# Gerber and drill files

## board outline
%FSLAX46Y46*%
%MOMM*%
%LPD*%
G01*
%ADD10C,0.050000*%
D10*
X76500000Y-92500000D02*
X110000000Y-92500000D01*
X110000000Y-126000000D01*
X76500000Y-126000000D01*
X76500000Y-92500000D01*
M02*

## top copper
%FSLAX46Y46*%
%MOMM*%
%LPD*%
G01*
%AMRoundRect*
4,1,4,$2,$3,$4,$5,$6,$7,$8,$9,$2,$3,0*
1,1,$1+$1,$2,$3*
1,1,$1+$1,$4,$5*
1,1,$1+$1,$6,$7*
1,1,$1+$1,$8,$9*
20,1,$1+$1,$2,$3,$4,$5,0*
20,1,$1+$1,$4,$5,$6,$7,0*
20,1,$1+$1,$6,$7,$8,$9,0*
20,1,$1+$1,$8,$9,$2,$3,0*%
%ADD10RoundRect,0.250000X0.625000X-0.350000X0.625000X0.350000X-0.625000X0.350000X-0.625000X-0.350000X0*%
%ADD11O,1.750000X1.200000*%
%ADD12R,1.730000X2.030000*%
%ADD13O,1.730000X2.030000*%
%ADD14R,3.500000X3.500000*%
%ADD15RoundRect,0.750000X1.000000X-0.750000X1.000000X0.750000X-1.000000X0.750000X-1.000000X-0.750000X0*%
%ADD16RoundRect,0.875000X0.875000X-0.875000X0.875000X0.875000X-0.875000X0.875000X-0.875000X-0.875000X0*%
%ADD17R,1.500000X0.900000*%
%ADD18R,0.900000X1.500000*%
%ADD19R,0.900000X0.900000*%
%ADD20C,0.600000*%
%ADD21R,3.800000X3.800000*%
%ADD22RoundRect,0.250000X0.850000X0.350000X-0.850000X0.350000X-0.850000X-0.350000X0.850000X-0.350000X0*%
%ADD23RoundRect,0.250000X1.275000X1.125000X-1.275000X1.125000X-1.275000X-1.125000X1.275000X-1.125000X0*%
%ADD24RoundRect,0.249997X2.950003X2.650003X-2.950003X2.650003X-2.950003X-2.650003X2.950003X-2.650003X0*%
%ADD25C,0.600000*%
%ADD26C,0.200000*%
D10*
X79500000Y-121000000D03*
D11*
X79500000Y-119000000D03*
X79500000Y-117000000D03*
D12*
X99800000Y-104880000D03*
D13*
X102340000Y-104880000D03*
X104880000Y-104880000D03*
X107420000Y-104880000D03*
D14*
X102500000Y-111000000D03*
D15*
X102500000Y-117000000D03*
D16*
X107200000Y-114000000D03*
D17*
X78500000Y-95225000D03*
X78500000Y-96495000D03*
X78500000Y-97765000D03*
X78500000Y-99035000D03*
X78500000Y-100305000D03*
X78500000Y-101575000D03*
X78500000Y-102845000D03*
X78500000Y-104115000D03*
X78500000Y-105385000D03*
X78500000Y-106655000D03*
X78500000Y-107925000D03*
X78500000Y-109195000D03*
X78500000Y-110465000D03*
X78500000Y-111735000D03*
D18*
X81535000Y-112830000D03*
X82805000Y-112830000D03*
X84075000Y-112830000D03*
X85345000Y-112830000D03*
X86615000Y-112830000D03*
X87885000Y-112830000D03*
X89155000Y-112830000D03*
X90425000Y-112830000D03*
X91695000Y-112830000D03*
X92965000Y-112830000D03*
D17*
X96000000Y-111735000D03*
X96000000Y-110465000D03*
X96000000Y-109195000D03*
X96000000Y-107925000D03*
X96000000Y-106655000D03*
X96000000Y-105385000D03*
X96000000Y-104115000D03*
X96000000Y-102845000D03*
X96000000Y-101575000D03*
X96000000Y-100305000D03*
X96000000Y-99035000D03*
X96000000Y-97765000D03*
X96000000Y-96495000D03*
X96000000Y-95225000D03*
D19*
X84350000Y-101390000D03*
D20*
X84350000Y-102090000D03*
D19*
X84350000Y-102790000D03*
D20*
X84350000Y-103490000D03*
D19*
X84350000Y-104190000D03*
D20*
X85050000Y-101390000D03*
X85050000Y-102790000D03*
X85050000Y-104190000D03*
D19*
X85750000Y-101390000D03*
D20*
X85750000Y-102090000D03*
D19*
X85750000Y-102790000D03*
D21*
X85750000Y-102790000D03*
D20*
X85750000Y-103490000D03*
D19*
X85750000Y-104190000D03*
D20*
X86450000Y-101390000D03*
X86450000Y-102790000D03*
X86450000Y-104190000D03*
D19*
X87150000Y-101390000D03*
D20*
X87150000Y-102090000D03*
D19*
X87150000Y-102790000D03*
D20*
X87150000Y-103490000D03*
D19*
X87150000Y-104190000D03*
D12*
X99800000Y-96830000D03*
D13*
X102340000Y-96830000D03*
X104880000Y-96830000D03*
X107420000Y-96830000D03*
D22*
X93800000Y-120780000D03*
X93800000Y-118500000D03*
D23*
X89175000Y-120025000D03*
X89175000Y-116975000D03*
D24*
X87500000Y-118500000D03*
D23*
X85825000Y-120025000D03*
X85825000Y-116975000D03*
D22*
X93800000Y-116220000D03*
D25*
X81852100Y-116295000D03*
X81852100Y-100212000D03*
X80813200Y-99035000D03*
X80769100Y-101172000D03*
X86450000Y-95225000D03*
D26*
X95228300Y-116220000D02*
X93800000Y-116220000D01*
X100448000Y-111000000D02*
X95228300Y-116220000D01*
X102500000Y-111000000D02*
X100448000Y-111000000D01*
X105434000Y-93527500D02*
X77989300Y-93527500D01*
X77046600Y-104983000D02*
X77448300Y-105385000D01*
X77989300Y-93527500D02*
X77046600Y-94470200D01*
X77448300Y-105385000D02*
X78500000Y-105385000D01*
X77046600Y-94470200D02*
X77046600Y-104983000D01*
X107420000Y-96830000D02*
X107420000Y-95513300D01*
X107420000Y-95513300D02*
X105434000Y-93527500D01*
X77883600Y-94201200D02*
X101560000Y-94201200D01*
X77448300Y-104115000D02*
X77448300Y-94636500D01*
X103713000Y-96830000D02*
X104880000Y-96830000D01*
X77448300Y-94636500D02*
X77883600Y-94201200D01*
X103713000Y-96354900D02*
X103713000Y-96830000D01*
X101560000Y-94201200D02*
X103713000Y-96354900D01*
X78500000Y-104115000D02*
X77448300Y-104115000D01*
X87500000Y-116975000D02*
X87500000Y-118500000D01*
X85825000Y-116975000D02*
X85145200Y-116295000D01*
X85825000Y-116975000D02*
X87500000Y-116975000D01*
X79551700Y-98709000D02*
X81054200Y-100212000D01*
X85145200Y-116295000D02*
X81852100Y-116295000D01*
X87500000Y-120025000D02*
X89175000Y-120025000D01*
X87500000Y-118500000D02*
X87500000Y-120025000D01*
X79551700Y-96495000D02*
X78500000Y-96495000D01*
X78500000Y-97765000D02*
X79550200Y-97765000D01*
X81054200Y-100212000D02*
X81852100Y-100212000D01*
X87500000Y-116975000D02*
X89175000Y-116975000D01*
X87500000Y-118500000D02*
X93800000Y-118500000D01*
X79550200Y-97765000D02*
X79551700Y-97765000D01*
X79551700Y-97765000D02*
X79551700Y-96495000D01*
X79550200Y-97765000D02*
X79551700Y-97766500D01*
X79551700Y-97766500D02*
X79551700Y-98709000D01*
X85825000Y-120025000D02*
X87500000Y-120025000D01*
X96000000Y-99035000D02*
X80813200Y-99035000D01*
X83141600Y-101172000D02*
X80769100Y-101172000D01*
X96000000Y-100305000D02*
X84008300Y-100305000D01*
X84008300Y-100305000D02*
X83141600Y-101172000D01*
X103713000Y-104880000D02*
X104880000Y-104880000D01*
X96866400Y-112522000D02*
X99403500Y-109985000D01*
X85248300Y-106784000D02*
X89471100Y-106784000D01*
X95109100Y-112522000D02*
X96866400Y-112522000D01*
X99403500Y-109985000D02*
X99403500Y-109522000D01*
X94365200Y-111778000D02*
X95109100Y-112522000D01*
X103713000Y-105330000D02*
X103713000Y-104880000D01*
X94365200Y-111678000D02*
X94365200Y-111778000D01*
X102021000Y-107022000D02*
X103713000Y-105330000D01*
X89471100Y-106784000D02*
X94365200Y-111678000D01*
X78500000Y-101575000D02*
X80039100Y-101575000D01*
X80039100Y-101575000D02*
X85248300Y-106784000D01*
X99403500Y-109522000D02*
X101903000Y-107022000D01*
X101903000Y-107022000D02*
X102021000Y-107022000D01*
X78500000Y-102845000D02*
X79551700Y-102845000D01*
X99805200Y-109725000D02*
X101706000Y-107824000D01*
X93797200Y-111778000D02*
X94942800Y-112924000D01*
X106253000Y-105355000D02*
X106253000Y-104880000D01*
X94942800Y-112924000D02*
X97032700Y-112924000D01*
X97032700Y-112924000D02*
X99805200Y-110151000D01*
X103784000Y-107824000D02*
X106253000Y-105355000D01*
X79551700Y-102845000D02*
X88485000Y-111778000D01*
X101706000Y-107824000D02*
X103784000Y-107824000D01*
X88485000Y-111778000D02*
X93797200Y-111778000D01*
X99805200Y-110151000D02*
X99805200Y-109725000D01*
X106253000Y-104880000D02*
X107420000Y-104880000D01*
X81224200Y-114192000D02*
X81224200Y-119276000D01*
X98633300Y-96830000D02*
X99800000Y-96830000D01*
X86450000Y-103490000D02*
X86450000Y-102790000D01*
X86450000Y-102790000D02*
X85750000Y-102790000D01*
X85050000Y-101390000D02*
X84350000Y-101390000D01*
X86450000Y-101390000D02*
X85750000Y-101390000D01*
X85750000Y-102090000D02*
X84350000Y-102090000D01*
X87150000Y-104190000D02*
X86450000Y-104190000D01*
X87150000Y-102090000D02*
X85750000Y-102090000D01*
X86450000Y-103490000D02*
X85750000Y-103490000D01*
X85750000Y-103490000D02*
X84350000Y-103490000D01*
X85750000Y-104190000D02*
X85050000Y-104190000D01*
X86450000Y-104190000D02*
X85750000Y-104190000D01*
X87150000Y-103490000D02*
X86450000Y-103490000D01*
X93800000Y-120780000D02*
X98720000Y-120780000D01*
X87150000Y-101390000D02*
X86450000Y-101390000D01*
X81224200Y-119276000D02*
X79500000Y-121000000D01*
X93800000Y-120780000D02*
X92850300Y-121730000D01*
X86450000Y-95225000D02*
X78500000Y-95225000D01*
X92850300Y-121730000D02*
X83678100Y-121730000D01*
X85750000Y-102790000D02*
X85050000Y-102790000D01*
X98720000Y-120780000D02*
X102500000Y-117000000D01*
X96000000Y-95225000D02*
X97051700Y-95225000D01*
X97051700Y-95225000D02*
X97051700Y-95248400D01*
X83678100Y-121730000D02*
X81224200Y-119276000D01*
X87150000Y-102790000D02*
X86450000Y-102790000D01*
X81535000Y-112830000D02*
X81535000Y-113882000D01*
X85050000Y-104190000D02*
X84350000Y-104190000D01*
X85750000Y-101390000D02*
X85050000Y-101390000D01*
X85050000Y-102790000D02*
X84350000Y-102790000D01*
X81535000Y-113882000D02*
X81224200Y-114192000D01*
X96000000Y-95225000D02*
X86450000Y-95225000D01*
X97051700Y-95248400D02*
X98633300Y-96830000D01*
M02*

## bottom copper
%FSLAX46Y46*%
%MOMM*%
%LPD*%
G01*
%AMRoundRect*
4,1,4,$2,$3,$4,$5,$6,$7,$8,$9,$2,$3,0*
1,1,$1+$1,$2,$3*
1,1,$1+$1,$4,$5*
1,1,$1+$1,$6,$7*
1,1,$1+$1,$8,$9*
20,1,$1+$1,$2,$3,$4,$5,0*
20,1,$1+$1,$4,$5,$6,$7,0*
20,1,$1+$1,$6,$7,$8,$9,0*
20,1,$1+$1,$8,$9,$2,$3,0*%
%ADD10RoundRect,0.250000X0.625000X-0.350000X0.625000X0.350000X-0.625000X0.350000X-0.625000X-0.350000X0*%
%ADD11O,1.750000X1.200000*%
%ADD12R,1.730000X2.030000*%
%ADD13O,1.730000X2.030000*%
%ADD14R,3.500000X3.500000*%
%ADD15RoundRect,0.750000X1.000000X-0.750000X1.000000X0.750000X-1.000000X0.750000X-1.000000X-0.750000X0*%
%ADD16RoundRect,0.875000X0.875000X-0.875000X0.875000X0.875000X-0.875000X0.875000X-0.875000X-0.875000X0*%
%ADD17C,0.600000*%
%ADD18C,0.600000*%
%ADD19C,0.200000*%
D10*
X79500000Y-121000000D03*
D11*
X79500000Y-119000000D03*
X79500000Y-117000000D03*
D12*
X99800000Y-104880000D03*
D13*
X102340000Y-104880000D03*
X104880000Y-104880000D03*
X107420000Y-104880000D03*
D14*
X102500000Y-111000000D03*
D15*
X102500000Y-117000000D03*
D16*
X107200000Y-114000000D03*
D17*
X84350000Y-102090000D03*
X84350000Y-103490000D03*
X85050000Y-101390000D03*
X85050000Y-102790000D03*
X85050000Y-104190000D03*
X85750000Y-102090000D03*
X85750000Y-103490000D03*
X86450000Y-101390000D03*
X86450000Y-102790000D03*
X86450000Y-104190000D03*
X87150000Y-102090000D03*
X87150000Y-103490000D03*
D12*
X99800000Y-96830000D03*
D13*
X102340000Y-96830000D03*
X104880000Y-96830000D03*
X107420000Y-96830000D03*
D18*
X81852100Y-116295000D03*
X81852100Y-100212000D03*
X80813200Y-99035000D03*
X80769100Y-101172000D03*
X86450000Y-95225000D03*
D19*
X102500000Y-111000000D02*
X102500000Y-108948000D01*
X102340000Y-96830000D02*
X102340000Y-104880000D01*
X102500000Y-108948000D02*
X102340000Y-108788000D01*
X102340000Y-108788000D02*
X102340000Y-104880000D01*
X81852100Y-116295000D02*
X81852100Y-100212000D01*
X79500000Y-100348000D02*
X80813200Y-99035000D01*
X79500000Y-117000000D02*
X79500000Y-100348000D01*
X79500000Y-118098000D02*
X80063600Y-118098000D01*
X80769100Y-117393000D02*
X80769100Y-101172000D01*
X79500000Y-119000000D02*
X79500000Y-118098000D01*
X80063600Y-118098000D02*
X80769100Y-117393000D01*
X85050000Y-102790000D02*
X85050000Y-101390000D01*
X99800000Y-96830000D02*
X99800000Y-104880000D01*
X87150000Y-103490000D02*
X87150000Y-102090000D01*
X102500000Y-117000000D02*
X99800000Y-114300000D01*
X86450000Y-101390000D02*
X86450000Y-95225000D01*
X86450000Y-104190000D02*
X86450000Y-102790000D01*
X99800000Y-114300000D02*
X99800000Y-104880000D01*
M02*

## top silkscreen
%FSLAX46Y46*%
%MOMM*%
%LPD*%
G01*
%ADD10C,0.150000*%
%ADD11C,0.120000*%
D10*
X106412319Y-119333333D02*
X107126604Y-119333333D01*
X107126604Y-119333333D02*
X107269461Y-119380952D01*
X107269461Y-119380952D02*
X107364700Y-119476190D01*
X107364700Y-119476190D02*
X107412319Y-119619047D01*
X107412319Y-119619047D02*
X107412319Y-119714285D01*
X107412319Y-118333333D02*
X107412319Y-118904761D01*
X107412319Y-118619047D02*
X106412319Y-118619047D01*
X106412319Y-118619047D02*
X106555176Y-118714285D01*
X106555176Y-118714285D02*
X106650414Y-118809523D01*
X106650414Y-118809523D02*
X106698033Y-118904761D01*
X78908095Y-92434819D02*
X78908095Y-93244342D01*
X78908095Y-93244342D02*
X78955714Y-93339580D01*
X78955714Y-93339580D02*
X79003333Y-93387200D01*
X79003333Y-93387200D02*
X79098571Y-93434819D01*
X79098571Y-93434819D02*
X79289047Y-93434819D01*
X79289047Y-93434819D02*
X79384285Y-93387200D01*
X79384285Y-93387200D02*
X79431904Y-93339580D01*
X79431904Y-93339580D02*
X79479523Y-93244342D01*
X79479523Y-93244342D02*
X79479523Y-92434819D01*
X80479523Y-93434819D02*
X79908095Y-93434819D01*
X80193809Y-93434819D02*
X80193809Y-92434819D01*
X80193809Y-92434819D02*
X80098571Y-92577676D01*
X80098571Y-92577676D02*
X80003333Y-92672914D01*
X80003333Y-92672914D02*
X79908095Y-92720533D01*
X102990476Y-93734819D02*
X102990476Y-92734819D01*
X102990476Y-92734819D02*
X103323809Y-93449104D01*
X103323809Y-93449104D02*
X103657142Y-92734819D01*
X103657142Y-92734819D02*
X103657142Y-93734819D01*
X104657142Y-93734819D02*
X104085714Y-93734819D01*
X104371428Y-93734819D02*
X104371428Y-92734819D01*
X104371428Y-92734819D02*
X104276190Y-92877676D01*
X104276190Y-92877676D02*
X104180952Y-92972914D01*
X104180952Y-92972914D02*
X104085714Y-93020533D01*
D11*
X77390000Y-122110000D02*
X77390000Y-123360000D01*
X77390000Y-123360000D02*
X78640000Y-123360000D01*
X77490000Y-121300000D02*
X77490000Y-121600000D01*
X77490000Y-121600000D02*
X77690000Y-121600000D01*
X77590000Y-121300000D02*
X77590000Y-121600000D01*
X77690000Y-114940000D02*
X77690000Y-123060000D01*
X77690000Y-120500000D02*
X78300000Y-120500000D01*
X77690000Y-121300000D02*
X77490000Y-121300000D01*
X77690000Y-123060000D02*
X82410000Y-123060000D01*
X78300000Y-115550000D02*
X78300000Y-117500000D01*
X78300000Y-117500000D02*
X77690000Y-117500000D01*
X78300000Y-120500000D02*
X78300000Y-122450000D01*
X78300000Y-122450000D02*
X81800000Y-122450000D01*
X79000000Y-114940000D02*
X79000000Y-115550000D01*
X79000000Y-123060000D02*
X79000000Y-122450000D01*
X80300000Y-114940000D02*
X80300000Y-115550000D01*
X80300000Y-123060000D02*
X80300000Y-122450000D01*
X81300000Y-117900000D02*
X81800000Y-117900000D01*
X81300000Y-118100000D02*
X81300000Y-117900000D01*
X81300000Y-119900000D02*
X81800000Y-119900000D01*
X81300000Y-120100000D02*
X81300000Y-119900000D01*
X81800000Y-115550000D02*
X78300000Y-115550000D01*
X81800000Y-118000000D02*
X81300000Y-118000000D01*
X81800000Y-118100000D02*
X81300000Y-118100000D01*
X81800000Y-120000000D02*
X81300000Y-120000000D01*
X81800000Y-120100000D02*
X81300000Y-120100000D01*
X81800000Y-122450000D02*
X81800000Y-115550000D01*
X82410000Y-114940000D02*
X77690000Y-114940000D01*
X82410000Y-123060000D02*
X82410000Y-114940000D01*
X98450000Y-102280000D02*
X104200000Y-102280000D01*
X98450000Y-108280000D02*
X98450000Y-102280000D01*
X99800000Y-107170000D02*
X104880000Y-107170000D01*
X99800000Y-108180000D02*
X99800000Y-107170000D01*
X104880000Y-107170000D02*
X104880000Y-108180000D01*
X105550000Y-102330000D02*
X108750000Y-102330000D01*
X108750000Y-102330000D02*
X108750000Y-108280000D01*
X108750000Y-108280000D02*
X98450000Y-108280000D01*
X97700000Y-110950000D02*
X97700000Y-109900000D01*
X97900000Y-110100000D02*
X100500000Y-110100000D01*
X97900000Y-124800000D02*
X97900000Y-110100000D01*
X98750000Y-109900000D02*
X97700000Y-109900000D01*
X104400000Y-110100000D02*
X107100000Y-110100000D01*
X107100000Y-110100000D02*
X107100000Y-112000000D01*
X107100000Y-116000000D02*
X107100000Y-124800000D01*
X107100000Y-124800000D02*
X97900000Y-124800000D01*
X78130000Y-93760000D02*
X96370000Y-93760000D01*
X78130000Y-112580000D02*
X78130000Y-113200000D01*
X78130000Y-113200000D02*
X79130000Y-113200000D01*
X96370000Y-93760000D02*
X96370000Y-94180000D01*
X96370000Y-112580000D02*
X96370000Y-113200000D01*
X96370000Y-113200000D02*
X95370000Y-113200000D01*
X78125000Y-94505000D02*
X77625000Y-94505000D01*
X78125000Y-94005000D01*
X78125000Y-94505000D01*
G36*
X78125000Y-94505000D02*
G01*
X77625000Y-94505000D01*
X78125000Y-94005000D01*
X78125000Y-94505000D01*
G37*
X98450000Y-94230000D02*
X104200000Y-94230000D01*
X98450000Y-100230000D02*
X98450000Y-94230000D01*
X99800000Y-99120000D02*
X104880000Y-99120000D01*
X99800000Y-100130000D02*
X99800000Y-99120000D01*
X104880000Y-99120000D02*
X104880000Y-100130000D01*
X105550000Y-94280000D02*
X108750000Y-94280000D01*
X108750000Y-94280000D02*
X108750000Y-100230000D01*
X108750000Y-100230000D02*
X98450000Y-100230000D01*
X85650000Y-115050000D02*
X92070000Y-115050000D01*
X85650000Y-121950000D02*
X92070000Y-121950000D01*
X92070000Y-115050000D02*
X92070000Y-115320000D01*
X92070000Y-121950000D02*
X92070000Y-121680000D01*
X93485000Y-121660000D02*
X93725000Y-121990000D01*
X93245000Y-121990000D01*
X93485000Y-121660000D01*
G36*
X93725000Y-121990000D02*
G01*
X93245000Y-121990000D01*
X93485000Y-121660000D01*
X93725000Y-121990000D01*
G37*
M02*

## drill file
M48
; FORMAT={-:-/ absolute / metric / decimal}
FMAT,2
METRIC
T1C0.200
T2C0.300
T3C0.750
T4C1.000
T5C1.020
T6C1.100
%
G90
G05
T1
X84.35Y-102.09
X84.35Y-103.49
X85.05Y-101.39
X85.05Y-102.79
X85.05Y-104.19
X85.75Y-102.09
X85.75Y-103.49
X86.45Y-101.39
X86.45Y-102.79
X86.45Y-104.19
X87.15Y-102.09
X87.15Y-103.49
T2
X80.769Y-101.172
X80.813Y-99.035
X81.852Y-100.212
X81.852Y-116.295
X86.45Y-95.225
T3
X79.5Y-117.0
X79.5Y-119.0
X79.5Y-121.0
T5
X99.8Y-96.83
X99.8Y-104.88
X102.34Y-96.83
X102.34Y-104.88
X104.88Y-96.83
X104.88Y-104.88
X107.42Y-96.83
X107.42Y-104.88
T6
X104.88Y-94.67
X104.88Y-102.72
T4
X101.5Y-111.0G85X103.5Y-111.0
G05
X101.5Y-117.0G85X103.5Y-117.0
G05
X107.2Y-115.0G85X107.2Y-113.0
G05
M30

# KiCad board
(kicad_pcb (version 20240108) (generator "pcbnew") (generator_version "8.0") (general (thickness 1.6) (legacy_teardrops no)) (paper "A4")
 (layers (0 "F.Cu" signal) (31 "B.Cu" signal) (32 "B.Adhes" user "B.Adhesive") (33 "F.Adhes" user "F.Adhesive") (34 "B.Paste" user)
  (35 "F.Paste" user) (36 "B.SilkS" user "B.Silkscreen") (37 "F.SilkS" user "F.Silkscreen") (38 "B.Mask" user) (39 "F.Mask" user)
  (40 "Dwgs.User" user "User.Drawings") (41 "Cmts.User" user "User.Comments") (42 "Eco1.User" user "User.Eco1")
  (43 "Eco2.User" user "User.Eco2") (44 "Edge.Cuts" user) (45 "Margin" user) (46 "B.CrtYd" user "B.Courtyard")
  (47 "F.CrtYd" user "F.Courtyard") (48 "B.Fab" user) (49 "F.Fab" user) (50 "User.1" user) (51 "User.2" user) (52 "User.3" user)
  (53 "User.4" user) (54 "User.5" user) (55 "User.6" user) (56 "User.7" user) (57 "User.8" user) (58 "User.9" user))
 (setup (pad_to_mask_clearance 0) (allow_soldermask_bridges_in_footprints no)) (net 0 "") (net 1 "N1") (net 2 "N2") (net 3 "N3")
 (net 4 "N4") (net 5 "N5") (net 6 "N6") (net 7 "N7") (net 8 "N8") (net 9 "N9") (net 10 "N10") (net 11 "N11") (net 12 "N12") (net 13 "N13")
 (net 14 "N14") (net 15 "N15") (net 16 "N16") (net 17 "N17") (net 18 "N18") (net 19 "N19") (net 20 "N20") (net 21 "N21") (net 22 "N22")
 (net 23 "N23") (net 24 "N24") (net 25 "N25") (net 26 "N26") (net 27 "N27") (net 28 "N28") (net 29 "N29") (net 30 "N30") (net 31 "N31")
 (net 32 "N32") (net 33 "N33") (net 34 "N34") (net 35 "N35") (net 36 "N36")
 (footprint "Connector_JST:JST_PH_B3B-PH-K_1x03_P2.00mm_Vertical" (layer "F.Cu") (at 79.5 121 90)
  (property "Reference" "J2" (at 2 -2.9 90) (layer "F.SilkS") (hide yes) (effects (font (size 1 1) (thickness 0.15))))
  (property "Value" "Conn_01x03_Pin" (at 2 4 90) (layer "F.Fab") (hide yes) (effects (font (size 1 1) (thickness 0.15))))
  (fp_line (start -1.11 -2.11) (end -2.36 -2.11) (stroke (width 0.12) (type solid)) (layer "F.SilkS"))
  (fp_line (start -2.36 -2.11) (end -2.36 -0.86) (stroke (width 0.12) (type solid)) (layer "F.SilkS"))
  (fp_line (start -0.3 -2.01) (end -0.6 -2.01) (stroke (width 0.12) (type solid)) (layer "F.SilkS"))
  (fp_line (start -0.6 -2.01) (end -0.6 -1.81) (stroke (width 0.12) (type solid)) (layer "F.SilkS"))
  (fp_line (start -0.3 -1.91) (end -0.6 -1.91) (stroke (width 0.12) (type solid)) (layer "F.SilkS"))
  (fp_line (start 6.06 -1.81) (end -2.06 -1.81) (stroke (width 0.12) (type solid)) (layer "F.SilkS"))
  (fp_line (start 0.5 -1.81) (end 0.5 -1.2) (stroke (width 0.12) (type solid)) (layer "F.SilkS"))
  (fp_line (start -0.3 -1.81) (end -0.3 -2.01) (stroke (width 0.12) (type solid)) (layer "F.SilkS"))
  (fp_line (start -2.06 -1.81) (end -2.06 2.91) (stroke (width 0.12) (type solid)) (layer "F.SilkS"))
  (fp_line (start 5.45 -1.2) (end 3.5 -1.2) (stroke (width 0.12) (type solid)) (layer "F.SilkS"))
  (fp_line (start 3.5 -1.2) (end 3.5 -1.81) (stroke (width 0.12) (type solid)) (layer "F.SilkS"))
  (fp_line (start 0.5 -1.2) (end -1.45 -1.2) (stroke (width 0.12) (type solid)) (layer "F.SilkS"))
  (fp_line (start -1.45 -1.2) (end -1.45 2.3) (stroke (width 0.12) (type solid)) (layer "F.SilkS"))
  (fp_line (start 6.06 -0.5) (end 5.45 -0.5) (stroke (width 0.12) (type solid)) (layer "F.SilkS"))
  (fp_line (start -2.06 -0.5) (end -1.45 -0.5) (stroke (width 0.12) (type solid)) (layer "F.SilkS"))
  (fp_line (start 6.06 0.8) (end 5.45 0.8) (stroke (width 0.12) (type solid)) (layer "F.SilkS"))
  (fp_line (start -2.06 0.8) (end -1.45 0.8) (stroke (width 0.12) (type solid)) (layer "F.SilkS"))
  (fp_line (start 3.1 1.8) (end 3.1 2.3) (stroke (width 0.12) (type solid)) (layer "F.SilkS"))
  (fp_line (start 2.9 1.8) (end 3.1 1.8) (stroke (width 0.12) (type solid)) (layer "F.SilkS"))
  (fp_line (start 1.1 1.8) (end 1.1 2.3) (stroke (width 0.12) (type solid)) (layer "F.SilkS"))
  (fp_line (start 0.9 1.8) (end 1.1 1.8) (stroke (width 0.12) (type solid)) (layer "F.SilkS"))
  (fp_line (start 5.45 2.3) (end 5.45 -1.2) (stroke (width 0.12) (type solid)) (layer "F.SilkS"))
  (fp_line (start 3 2.3) (end 3 1.8) (stroke (width 0.12) (type solid)) (layer "F.SilkS"))
  (fp_line (start 2.9 2.3) (end 2.9 1.8) (stroke (width 0.12) (type solid)) (layer "F.SilkS"))
  (fp_line (start 1 2.3) (end 1 1.8) (stroke (width 0.12) (type solid)) (layer "F.SilkS"))
  (fp_line (start 0.9 2.3) (end 0.9 1.8) (stroke (width 0.12) (type solid)) (layer "F.SilkS"))
  (fp_line (start -1.45 2.3) (end 5.45 2.3) (stroke (width 0.12) (type solid)) (layer "F.SilkS"))
  (fp_line (start 6.06 2.91) (end 6.06 -1.81) (stroke (width 0.12) (type solid)) (layer "F.SilkS"))
  (fp_line (start -2.06 2.91) (end 6.06 2.91) (stroke (width 0.12) (type solid)) (layer "F.SilkS"))
  (pad "1" thru_hole roundrect (at 0 0 90) (size 1.2 1.75) (drill 0.75) (layers "*.Cu" "*.Mask") (remove_unused_layers no)
   (roundrect_rratio 0.208333) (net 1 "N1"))
  (pad "2" thru_hole oval (at 2 0 90) (size 1.2 1.75) (drill 0.75) (layers "*.Cu" "*.Mask") (remove_unused_layers no) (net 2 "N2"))
  (pad "3" thru_hole oval (at 4 0 90) (size 1.2 1.75) (drill 0.75) (layers "*.Cu" "*.Mask") (remove_unused_layers no) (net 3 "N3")))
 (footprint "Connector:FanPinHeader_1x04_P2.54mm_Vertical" (layer "F.Cu") (at 99.8 104.88)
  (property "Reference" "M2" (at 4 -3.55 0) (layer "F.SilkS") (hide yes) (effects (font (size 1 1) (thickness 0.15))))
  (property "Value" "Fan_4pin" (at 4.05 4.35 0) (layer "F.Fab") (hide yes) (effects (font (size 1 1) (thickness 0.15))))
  (fp_line (start -1.35 -2.6) (end 4.4 -2.6) (stroke (width 0.12) (type solid)) (layer "F.SilkS"))
  (fp_line (start -1.35 3.4) (end -1.35 -2.6) (stroke (width 0.12) (type solid)) (layer "F.SilkS"))
  (fp_line (start 0 2.29) (end 5.08 2.29) (stroke (width 0.12) (type solid)) (layer "F.SilkS"))
  (fp_line (start 0 3.3) (end 0 2.29) (stroke (width 0.12) (type solid)) (layer "F.SilkS"))
  (fp_line (start 5.08 2.29) (end 5.08 3.3) (stroke (width 0.12) (type solid)) (layer "F.SilkS"))
  (fp_line (start 5.75 -2.55) (end 8.95 -2.55) (stroke (width 0.12) (type solid)) (layer "F.SilkS"))
  (fp_line (start 8.95 -2.55) (end 8.95 3.4) (stroke (width 0.12) (type solid)) (layer "F.SilkS"))
  (fp_line (start 8.95 3.4) (end -1.35 3.4) (stroke (width 0.12) (type solid)) (layer "F.SilkS"))
  (pad "" np_thru_hole circle (at 5.08 -2.16 90) (size 1.1 1.1) (drill 1.1) (layers "*.Cu" "*.Mask"))
  (pad "1" thru_hole rect (at 0 0 90) (size 2.03 1.73) (drill 1.02) (layers "*.Cu" "*.Mask") (remove_unused_layers no) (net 1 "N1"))
  (pad "2" thru_hole oval (at 2.54 0 90) (size 2.03 1.73) (drill 1.02) (layers "*.Cu" "*.Mask") (remove_unused_layers no) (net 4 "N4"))
  (pad "3" thru_hole oval (at 5.08 0 90) (size 2.03 1.73) (drill 1.02) (layers "*.Cu" "*.Mask") (remove_unused_layers no) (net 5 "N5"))
  (pad "4" thru_hole oval (at 7.62 0 90) (size 2.03 1.73) (drill 1.02) (layers "*.Cu" "*.Mask") (remove_unused_layers no) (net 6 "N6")))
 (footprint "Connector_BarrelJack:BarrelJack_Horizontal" (layer "F.Cu") (at 102.5 111 90)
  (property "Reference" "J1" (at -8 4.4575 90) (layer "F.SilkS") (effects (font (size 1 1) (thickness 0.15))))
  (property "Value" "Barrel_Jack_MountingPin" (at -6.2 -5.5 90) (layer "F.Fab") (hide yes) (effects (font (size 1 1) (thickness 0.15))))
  (fp_line (start 0.05 -4.8) (end 1.1 -4.8) (stroke (width 0.12) (type solid)) (layer "F.SilkS"))
  (fp_line (start 0.9 -4.6) (end 0.9 -2) (stroke (width 0.12) (type solid)) (layer "F.SilkS"))
  (fp_line (start -13.8 -4.6) (end 0.9 -4.6) (stroke (width 0.12) (type solid)) (layer "F.SilkS"))
  (fp_line (start 1.1 -3.75) (end 1.1 -4.8) (stroke (width 0.12) (type solid)) (layer "F.SilkS"))
  (fp_line (start 0.9 1.9) (end 0.9 4.6) (stroke (width 0.12) (type solid)) (layer "F.SilkS"))
  (fp_line (start 0.9 4.6) (end -1 4.6) (stroke (width 0.12) (type solid)) (layer "F.SilkS"))
  (fp_line (start -5 4.6) (end -13.8 4.6) (stroke (width 0.12) (type solid)) (layer "F.SilkS"))
  (fp_line (start -13.8 4.6) (end -13.8 -4.6) (stroke (width 0.12) (type solid)) (layer "F.SilkS"))
  (pad "1" thru_hole rect (at 0 0 90) (size 3.5 3.5) (drill oval 1 3) (layers "*.Cu" "*.Mask") (remove_unused_layers no) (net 4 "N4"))
  (pad "2" thru_hole roundrect (at -6 0 90) (size 3 3.5) (drill oval 1 3) (layers "*.Cu" "*.Mask") (remove_unused_layers no)
   (roundrect_rratio 0.25) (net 1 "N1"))
  (pad "3" thru_hole roundrect (at -3 4.7 90) (size 3.5 3.5) (drill oval 3 1) (layers "*.Cu" "*.Mask") (remove_unused_layers no)
   (roundrect_rratio 0.25)))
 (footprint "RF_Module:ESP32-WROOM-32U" (layer "F.Cu") (at 87.25 103.48)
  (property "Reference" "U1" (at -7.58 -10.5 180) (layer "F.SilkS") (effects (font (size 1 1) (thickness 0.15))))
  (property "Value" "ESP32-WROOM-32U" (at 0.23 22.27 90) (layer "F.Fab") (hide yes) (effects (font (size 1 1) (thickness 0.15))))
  (fp_line (start -9.12 -9.72) (end 9.12 -9.72) (stroke (width 0.12) (type solid)) (layer "F.SilkS"))
  (fp_line (start -9.12 9.1) (end -9.12 9.72) (stroke (width 0.12) (type solid)) (layer "F.SilkS"))
  (fp_line (start -9.12 9.72) (end -8.12 9.72) (stroke (width 0.12) (type solid)) (layer "F.SilkS"))
  (fp_line (start 9.12 -9.72) (end 9.12 -9.3) (stroke (width 0.12) (type solid)) (layer "F.SilkS"))
  (fp_line (start 9.12 9.1) (end 9.12 9.72) (stroke (width 0.12) (type solid)) (layer "F.SilkS"))
  (fp_line (start 9.12 9.72) (end 8.12 9.72) (stroke (width 0.12) (type solid)) (layer "F.SilkS"))
  (fp_poly
   (pts (xy -9.125 -8.975) (xy -9.625 -8.975) (xy -9.125 -9.475) (xy -9.125 -8.975)) (stroke (width 0.12) (type solid)) (fill solid)
   (layer "F.SilkS"))
  (pad "1" smd rect (at -8.75 -8.255) (size 1.5 0.9) (layers "F.Cu" "F.Paste" "F.Mask") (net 1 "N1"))
  (pad "2" smd rect (at -8.75 -6.985) (size 1.5 0.9) (layers "F.Cu" "F.Paste" "F.Mask") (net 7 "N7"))
  (pad "3" smd rect (at -8.75 -5.715) (size 1.5 0.9) (layers "F.Cu" "F.Paste" "F.Mask") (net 7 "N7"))
  (pad "4" smd rect (at -8.75 -4.445) (size 1.5 0.9) (layers "F.Cu" "F.Paste" "F.Mask") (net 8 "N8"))
  (pad "5" smd rect (at -8.75 -3.175) (size 1.5 0.9) (layers "F.Cu" "F.Paste" "F.Mask") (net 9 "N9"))
  (pad "6" smd rect (at -8.75 -1.905) (size 1.5 0.9) (layers "F.Cu" "F.Paste" "F.Mask") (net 5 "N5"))
  (pad "7" smd rect (at -8.75 -0.635) (size 1.5 0.9) (layers "F.Cu" "F.Paste" "F.Mask") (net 6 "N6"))
  (pad "8" smd rect (at -8.75 0.635) (size 1.5 0.9) (layers "F.Cu" "F.Paste" "F.Mask") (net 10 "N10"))
  (pad "9" smd rect (at -8.75 1.905) (size 1.5 0.9) (layers "F.Cu" "F.Paste" "F.Mask") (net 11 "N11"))
  (pad "10" smd rect (at -8.75 3.175) (size 1.5 0.9) (layers "F.Cu" "F.Paste" "F.Mask") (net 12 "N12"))
  (pad "11" smd rect (at -8.75 4.445) (size 1.5 0.9) (layers "F.Cu" "F.Paste" "F.Mask") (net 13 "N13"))
  (pad "12" smd rect (at -8.75 5.715) (size 1.5 0.9) (layers "F.Cu" "F.Paste" "F.Mask") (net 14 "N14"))
  (pad "13" smd rect (at -8.75 6.985) (size 1.5 0.9) (layers "F.Cu" "F.Paste" "F.Mask") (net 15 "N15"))
  (pad "14" smd rect (at -8.75 8.255) (size 1.5 0.9) (layers "F.Cu" "F.Paste" "F.Mask") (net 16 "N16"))
  (pad "15" smd rect (at -5.715 9.35 90) (size 1.5 0.9) (layers "F.Cu" "F.Paste" "F.Mask") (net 1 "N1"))
  (pad "16" smd rect (at -4.445 9.35 90) (size 1.5 0.9) (layers "F.Cu" "F.Paste" "F.Mask") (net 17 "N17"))
  (pad "17" smd rect (at -3.175 9.35 90) (size 1.5 0.9) (layers "F.Cu" "F.Paste" "F.Mask") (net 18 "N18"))
  (pad "18" smd rect (at -1.905 9.35 90) (size 1.5 0.9) (layers "F.Cu" "F.Paste" "F.Mask") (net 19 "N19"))
  (pad "19" smd rect (at -0.635 9.35 90) (size 1.5 0.9) (layers "F.Cu" "F.Paste" "F.Mask") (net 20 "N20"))
  (pad "20" smd rect (at 0.635 9.35 90) (size 1.5 0.9) (layers "F.Cu" "F.Paste" "F.Mask") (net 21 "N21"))
  (pad "21" smd rect (at 1.905 9.35 90) (size 1.5 0.9) (layers "F.Cu" "F.Paste" "F.Mask") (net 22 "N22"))
  (pad "22" smd rect (at 3.175 9.35 90) (size 1.5 0.9) (layers "F.Cu" "F.Paste" "F.Mask") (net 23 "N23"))
  (pad "23" smd rect (at 4.445 9.35 90) (size 1.5 0.9) (layers "F.Cu" "F.Paste" "F.Mask") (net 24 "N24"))
  (pad "24" smd rect (at 5.715 9.35 90) (size 1.5 0.9) (layers "F.Cu" "F.Paste" "F.Mask") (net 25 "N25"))
  (pad "25" smd rect (at 8.75 8.255) (size 1.5 0.9) (layers "F.Cu" "F.Paste" "F.Mask") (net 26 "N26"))
  (pad "26" smd rect (at 8.75 6.985) (size 1.5 0.9) (layers "F.Cu" "F.Paste" "F.Mask") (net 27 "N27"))
  (pad "27" smd rect (at 8.75 5.715) (size 1.5 0.9) (layers "F.Cu" "F.Paste" "F.Mask") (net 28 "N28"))
  (pad "28" smd rect (at 8.75 4.445) (size 1.5 0.9) (layers "F.Cu" "F.Paste" "F.Mask") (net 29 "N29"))
  (pad "29" smd rect (at 8.75 3.175) (size 1.5 0.9) (layers "F.Cu" "F.Paste" "F.Mask") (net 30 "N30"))
  (pad "30" smd rect (at 8.75 1.905) (size 1.5 0.9) (layers "F.Cu" "F.Paste" "F.Mask") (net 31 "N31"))
  (pad "31" smd rect (at 8.75 0.635) (size 1.5 0.9) (layers "F.Cu" "F.Paste" "F.Mask") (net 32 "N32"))
  (pad "32" smd rect (at 8.75 -0.635) (size 1.5 0.9) (layers "F.Cu" "F.Paste" "F.Mask") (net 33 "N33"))
  (pad "33" smd rect (at 8.75 -1.905) (size 1.5 0.9) (layers "F.Cu" "F.Paste" "F.Mask") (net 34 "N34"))
  (pad "34" smd rect (at 8.75 -3.175) (size 1.5 0.9) (layers "F.Cu" "F.Paste" "F.Mask") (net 2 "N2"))
  (pad "35" smd rect (at 8.75 -4.445) (size 1.5 0.9) (layers "F.Cu" "F.Paste" "F.Mask") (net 3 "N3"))
  (pad "36" smd rect (at 8.75 -5.715) (size 1.5 0.9) (layers "F.Cu" "F.Paste" "F.Mask") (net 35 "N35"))
  (pad "37" smd rect (at 8.75 -6.985) (size 1.5 0.9) (layers "F.Cu" "F.Paste" "F.Mask") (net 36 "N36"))
  (pad "38" smd rect (at 8.75 -8.255) (size 1.5 0.9) (layers "F.Cu" "F.Paste" "F.Mask") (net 1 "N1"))
  (pad "39" smd rect (at -2.9 -2.09) (size 0.9 0.9) (layers "F.Cu" "F.Paste") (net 1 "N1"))
  (pad "39" thru_hole circle (at -2.9 -1.39) (size 0.6 0.6) (drill 0.2) (layers "*.Cu" "F.Mask") (remove_unused_layers no) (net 1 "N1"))
  (pad "39" smd rect (at -2.9 -0.69) (size 0.9 0.9) (layers "F.Cu" "F.Paste") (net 1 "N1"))
  (pad "39" thru_hole circle (at -2.9 0.01) (size 0.6 0.6) (drill 0.2) (layers "*.Cu" "F.Mask") (remove_unused_layers no) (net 1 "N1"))
  (pad "39" smd rect (at -2.9 0.71) (size 0.9 0.9) (layers "F.Cu" "F.Paste") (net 1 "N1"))
  (pad "39" thru_hole circle (at -2.2 -2.09) (size 0.6 0.6) (drill 0.2) (layers "*.Cu" "F.Mask") (remove_unused_layers no) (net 1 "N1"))
  (pad "39" thru_hole circle (at -2.2 -0.69) (size 0.6 0.6) (drill 0.2) (layers "*.Cu" "F.Mask") (remove_unused_layers no) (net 1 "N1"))
  (pad "39" thru_hole circle (at -2.2 0.71) (size 0.6 0.6) (drill 0.2) (layers "*.Cu" "F.Mask") (remove_unused_layers no) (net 1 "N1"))
  (pad "39" smd rect (at -1.5 -2.09) (size 0.9 0.9) (layers "F.Cu" "F.Paste") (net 1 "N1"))
  (pad "39" thru_hole circle (at -1.5 -1.39) (size 0.6 0.6) (drill 0.2) (layers "*.Cu" "F.Mask") (remove_unused_layers no) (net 1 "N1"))
  (pad "39" smd rect (at -1.5 -0.69) (size 0.9 0.9) (layers "F.Cu" "F.Paste") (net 1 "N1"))
  (pad "39" smd rect (at -1.5 -0.69) (size 3.8 3.8) (layers "F.Cu" "F.Mask") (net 1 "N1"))
  (pad "39" thru_hole circle (at -1.5 0.01) (size 0.6 0.6) (drill 0.2) (layers "*.Cu" "F.Mask") (remove_unused_layers no) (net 1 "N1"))
  (pad "39" smd rect (at -1.5 0.71) (size 0.9 0.9) (layers "F.Cu" "F.Paste") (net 1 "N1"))
  (pad "39" thru_hole circle (at -0.8 -2.09) (size 0.6 0.6) (drill 0.2) (layers "*.Cu" "F.Mask") (remove_unused_layers no) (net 1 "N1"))
  (pad "39" thru_hole circle (at -0.8 -0.69) (size 0.6 0.6) (drill 0.2) (layers "*.Cu" "F.Mask") (remove_unused_layers no) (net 1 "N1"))
  (pad "39" thru_hole circle (at -0.8 0.71) (size 0.6 0.6) (drill 0.2) (layers "*.Cu" "F.Mask") (remove_unused_layers no) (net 1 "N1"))
  (pad "39" smd rect (at -0.1 -2.09) (size 0.9 0.9) (layers "F.Cu" "F.Paste") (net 1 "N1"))
  (pad "39" thru_hole circle (at -0.1 -1.39) (size 0.6 0.6) (drill 0.2) (layers "*.Cu" "F.Mask") (remove_unused_layers no) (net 1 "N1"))
  (pad "39" smd rect (at -0.1 -0.69) (size 0.9 0.9) (layers "F.Cu" "F.Paste") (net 1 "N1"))
  (pad "39" thru_hole circle (at -0.1 0.01) (size 0.6 0.6) (drill 0.2) (layers "*.Cu" "F.Mask") (remove_unused_layers no) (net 1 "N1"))
  (pad "39" smd rect (at -0.1 0.71) (size 0.9 0.9) (layers "F.Cu" "F.Paste") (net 1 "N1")))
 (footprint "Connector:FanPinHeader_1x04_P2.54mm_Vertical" (layer "F.Cu") (at 99.8 96.83)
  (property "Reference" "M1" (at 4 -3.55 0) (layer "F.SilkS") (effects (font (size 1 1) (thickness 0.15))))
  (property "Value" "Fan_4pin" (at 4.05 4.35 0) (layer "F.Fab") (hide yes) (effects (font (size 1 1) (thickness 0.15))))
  (fp_line (start -1.35 -2.6) (end 4.4 -2.6) (stroke (width 0.12) (type solid)) (layer "F.SilkS"))
  (fp_line (start -1.35 3.4) (end -1.35 -2.6) (stroke (width 0.12) (type solid)) (layer "F.SilkS"))
  (fp_line (start 0 2.29) (end 5.08 2.29) (stroke (width 0.12) (type solid)) (layer "F.SilkS"))
  (fp_line (start 0 3.3) (end 0 2.29) (stroke (width 0.12) (type solid)) (layer "F.SilkS"))
  (fp_line (start 5.08 2.29) (end 5.08 3.3) (stroke (width 0.12) (type solid)) (layer "F.SilkS"))
  (fp_line (start 5.75 -2.55) (end 8.95 -2.55) (stroke (width 0.12) (type solid)) (layer "F.SilkS"))
  (fp_line (start 8.95 -2.55) (end 8.95 3.4) (stroke (width 0.12) (type solid)) (layer "F.SilkS"))
  (fp_line (start 8.95 3.4) (end -1.35 3.4) (stroke (width 0.12) (type solid)) (layer "F.SilkS"))
  (pad "" np_thru_hole circle (at 5.08 -2.16 90) (size 1.1 1.1) (drill 1.1) (layers "*.Cu" "*.Mask"))
  (pad "1" thru_hole rect (at 0 0 90) (size 2.03 1.73) (drill 1.02) (layers "*.Cu" "*.Mask") (remove_unused_layers no) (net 1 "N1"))
  (pad "2" thru_hole oval (at 2.54 0 90) (size 2.03 1.73) (drill 1.02) (layers "*.Cu" "*.Mask") (remove_unused_layers no) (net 4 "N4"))
  (pad "3" thru_hole oval (at 5.08 0 90) (size 2.03 1.73) (drill 1.02) (layers "*.Cu" "*.Mask") (remove_unused_layers no) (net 10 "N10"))
  (pad "4" thru_hole oval (at 7.62 0 90) (size 2.03 1.73) (drill 1.02) (layers "*.Cu" "*.Mask") (remove_unused_layers no) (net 11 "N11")))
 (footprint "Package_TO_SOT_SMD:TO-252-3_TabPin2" (layer "F.Cu") (at 88.76 118.5 180)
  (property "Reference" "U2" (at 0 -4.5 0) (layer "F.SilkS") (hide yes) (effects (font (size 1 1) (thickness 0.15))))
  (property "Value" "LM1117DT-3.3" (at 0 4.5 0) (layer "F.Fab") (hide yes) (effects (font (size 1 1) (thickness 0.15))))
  (fp_line (start 3.11 3.45) (end -3.31 3.45) (stroke (width 0.12) (type solid)) (layer "F.SilkS"))
  (fp_line (start 3.11 -3.45) (end -3.31 -3.45) (stroke (width 0.12) (type solid)) (layer "F.SilkS"))
  (fp_line (start -3.31 3.45) (end -3.31 3.18) (stroke (width 0.12) (type solid)) (layer "F.SilkS"))
  (fp_line (start -3.31 -3.45) (end -3.31 -3.18) (stroke (width 0.12) (type solid)) (layer "F.SilkS"))
  (fp_poly
   (pts (xy -4.725 -3.16) (xy -4.965 -3.49) (xy -4.485 -3.49) (xy -4.725 -3.16)) (stroke (width 0.12) (type solid)) (fill solid)
   (layer "F.SilkS"))
  (pad "1" smd roundrect (at -5.04 -2.28 180) (size 2.2 1.2) (layers "F.Cu" "F.Paste" "F.Mask") (roundrect_rratio 0.208333) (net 1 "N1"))
  (pad "2" smd roundrect (at -5.04 0 180) (size 2.2 1.2) (layers "F.Cu" "F.Paste" "F.Mask") (roundrect_rratio 0.208333) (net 7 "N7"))
  (pad "2" smd roundrect (at -0.415 -1.525 180) (size 3.05 2.75) (layers "F.Cu" "F.Paste") (roundrect_rratio 0.090909) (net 7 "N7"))
  (pad "2" smd roundrect (at -0.415 1.525 180) (size 3.05 2.75) (layers "F.Cu" "F.Paste") (roundrect_rratio 0.090909) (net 7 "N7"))
  (pad "2" smd roundrect (at 1.26 0 180) (size 6.4 5.8) (layers "F.Cu" "F.Mask") (roundrect_rratio 0.043103) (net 7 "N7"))
  (pad "2" smd roundrect (at 2.935 -1.525 180) (size 3.05 2.75) (layers "F.Cu" "F.Paste") (roundrect_rratio 0.090909) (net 7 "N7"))
  (pad "2" smd roundrect (at 2.935 1.525 180) (size 3.05 2.75) (layers "F.Cu" "F.Paste") (roundrect_rratio 0.090909) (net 7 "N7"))
  (pad "3" smd roundrect (at -5.04 2.28 180) (size 2.2 1.2) (layers "F.Cu" "F.Paste" "F.Mask") (roundrect_rratio 0.208333) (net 4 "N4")))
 (gr_rect (start 76.5 92.5) (end 110 126) (stroke (width 0.05) (type default)) (fill none) (layer "Edge.Cuts"))
 (segment (start 95.2283 116.22) (end 93.8 116.22) (width 0.2) (layer "F.Cu") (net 4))
 (segment (start 100.448 111) (end 95.2283 116.22) (width 0.2) (layer "F.Cu") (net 4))
 (segment (start 102.5 111) (end 100.448 111) (width 0.2) (layer "F.Cu") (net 4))
 (segment (start 102.5 111) (end 102.5 108.948) (width 0.2) (layer "B.Cu") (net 4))
 (segment (start 102.34 96.83) (end 102.34 104.88) (width 0.2) (layer "B.Cu") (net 4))
 (segment (start 102.5 108.948) (end 102.34 108.788) (width 0.2) (layer "B.Cu") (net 4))
 (segment (start 102.34 108.788) (end 102.34 104.88) (width 0.2) (layer "B.Cu") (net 4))
 (segment (start 105.434 93.5275) (end 77.9893 93.5275) (width 0.2) (layer "F.Cu") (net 11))
 (segment (start 77.0466 104.983) (end 77.4483 105.385) (width 0.2) (layer "F.Cu") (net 11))
 (segment (start 77.9893 93.5275) (end 77.0466 94.4702) (width 0.2) (layer "F.Cu") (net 11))
 (segment (start 77.4483 105.385) (end 78.5 105.385) (width 0.2) (layer "F.Cu") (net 11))
 (segment (start 77.0466 94.4702) (end 77.0466 104.983) (width 0.2) (layer "F.Cu") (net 11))
 (segment (start 107.42 96.83) (end 107.42 95.5133) (width 0.2) (layer "F.Cu") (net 11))
 (segment (start 107.42 95.5133) (end 105.434 93.5275) (width 0.2) (layer "F.Cu") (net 11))
 (segment (start 77.8836 94.2012) (end 101.56 94.2012) (width 0.2) (layer "F.Cu") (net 10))
 (segment (start 77.4483 104.115) (end 77.4483 94.6365) (width 0.2) (layer "F.Cu") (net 10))
 (segment (start 103.713 96.83) (end 104.88 96.83) (width 0.2) (layer "F.Cu") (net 10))
 (segment (start 77.4483 94.6365) (end 77.8836 94.2012) (width 0.2) (layer "F.Cu") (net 10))
 (segment (start 103.713 96.3549) (end 103.713 96.83) (width 0.2) (layer "F.Cu") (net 10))
 (segment (start 101.56 94.2012) (end 103.713 96.3549) (width 0.2) (layer "F.Cu") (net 10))
 (segment (start 78.5 104.115) (end 77.4483 104.115) (width 0.2) (layer "F.Cu") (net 10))
 (segment (start 87.5 116.975) (end 87.5 118.5) (width 0.2) (layer "F.Cu") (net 7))
 (segment (start 85.825 116.975) (end 85.1452 116.295) (width 0.2) (layer "F.Cu") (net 7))
 (segment (start 85.825 116.975) (end 87.5 116.975) (width 0.2) (layer "F.Cu") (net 7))
 (segment (start 79.5517 98.709) (end 81.0542 100.212) (width 0.2) (layer "F.Cu") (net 7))
 (segment (start 85.1452 116.295) (end 81.8521 116.295) (width 0.2) (layer "F.Cu") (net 7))
 (segment (start 87.5 120.025) (end 89.175 120.025) (width 0.2) (layer "F.Cu") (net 7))
 (segment (start 87.5 118.5) (end 87.5 120.025) (width 0.2) (layer "F.Cu") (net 7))
 (segment (start 79.5517 96.495) (end 78.5 96.495) (width 0.2) (layer "F.Cu") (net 7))
 (segment (start 78.5 97.765) (end 79.5502 97.765) (width 0.2) (layer "F.Cu") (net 7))
 (segment (start 81.0542 100.212) (end 81.8521 100.212) (width 0.2) (layer "F.Cu") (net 7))
 (segment (start 87.5 116.975) (end 89.175 116.975) (width 0.2) (layer "F.Cu") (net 7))
 (segment (start 87.5 118.5) (end 93.8 118.5) (width 0.2) (layer "F.Cu") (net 7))
 (segment (start 79.5502 97.765) (end 79.5517 97.765) (width 0.2) (layer "F.Cu") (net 7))
 (segment (start 79.5517 97.765) (end 79.5517 96.495) (width 0.2) (layer "F.Cu") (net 7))
 (segment (start 79.5502 97.765) (end 79.5517 97.7665) (width 0.2) (layer "F.Cu") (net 7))
 (segment (start 79.5517 97.7665) (end 79.5517 98.709) (width 0.2) (layer "F.Cu") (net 7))
 (segment (start 85.825 120.025) (end 87.5 120.025) (width 0.2) (layer "F.Cu") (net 7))
 (via (at 81.8521 116.295) (size 0.6) (drill 0.3) (layers "F.Cu" "B.Cu") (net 7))
 (via (at 81.8521 100.212) (size 0.6) (drill 0.3) (layers "F.Cu" "B.Cu") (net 7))
 (segment (start 81.8521 116.295) (end 81.8521 100.212) (width 0.2) (layer "B.Cu") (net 7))
 (segment (start 96 99.035) (end 80.8132 99.035) (width 0.2) (layer "F.Cu") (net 3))
 (via (at 80.8132 99.035) (size 0.6) (drill 0.3) (layers "F.Cu" "B.Cu") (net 3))
 (segment (start 79.5 100.348) (end 80.8132 99.035) (width 0.2) (layer "B.Cu") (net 3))
 (segment (start 79.5 117) (end 79.5 100.348) (width 0.2) (layer "B.Cu") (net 3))
 (segment (start 83.1416 101.172) (end 80.7691 101.172) (width 0.2) (layer "F.Cu") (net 2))
 (segment (start 96 100.305) (end 84.0083 100.305) (width 0.2) (layer "F.Cu") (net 2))
 (segment (start 84.0083 100.305) (end 83.1416 101.172) (width 0.2) (layer "F.Cu") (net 2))
 (via (at 80.7691 101.172) (size 0.6) (drill 0.3) (layers "F.Cu" "B.Cu") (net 2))
 (segment (start 79.5 118.098) (end 80.0636 118.098) (width 0.2) (layer "B.Cu") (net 2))
 (segment (start 80.7691 117.393) (end 80.7691 101.172) (width 0.2) (layer "B.Cu") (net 2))
 (segment (start 79.5 119) (end 79.5 118.098) (width 0.2) (layer "B.Cu") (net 2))
 (segment (start 80.0636 118.098) (end 80.7691 117.393) (width 0.2) (layer "B.Cu") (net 2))
 (segment (start 103.713 104.88) (end 104.88 104.88) (width 0.2) (layer "F.Cu") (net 5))
 (segment (start 96.8664 112.522) (end 99.4035 109.985) (width 0.2) (layer "F.Cu") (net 5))
 (segment (start 85.2483 106.784) (end 89.4711 106.784) (width 0.2) (layer "F.Cu") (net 5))
 (segment (start 95.1091 112.522) (end 96.8664 112.522) (width 0.2) (layer "F.Cu") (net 5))
 (segment (start 99.4035 109.985) (end 99.4035 109.522) (width 0.2) (layer "F.Cu") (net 5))
 (segment (start 94.3652 111.778) (end 95.1091 112.522) (width 0.2) (layer "F.Cu") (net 5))
 (segment (start 103.713 105.33) (end 103.713 104.88) (width 0.2) (layer "F.Cu") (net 5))
 (segment (start 94.3652 111.678) (end 94.3652 111.778) (width 0.2) (layer "F.Cu") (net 5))
 (segment (start 102.021 107.022) (end 103.713 105.33) (width 0.2) (layer "F.Cu") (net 5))
 (segment (start 89.4711 106.784) (end 94.3652 111.678) (width 0.2) (layer "F.Cu") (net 5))
 (segment (start 78.5 101.575) (end 80.0391 101.575) (width 0.2) (layer "F.Cu") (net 5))
 (segment (start 80.0391 101.575) (end 85.2483 106.784) (width 0.2) (layer "F.Cu") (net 5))
 (segment (start 99.4035 109.522) (end 101.903 107.022) (width 0.2) (layer "F.Cu") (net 5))
 (segment (start 101.903 107.022) (end 102.021 107.022) (width 0.2) (layer "F.Cu") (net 5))
 (segment (start 78.5 102.845) (end 79.5517 102.845) (width 0.2) (layer "F.Cu") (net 6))
 (segment (start 99.8052 109.725) (end 101.706 107.824) (width 0.2) (layer "F.Cu") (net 6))
 (segment (start 93.7972 111.778) (end 94.9428 112.924) (width 0.2) (layer "F.Cu") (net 6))
 (segment (start 106.253 105.355) (end 106.253 104.88) (width 0.2) (layer "F.Cu") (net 6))
 (segment (start 94.9428 112.924) (end 97.0327 112.924) (width 0.2) (layer "F.Cu") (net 6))
 (segment (start 97.0327 112.924) (end 99.8052 110.151) (width 0.2) (layer "F.Cu") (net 6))
 (segment (start 103.784 107.824) (end 106.253 105.355) (width 0.2) (layer "F.Cu") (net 6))
 (segment (start 79.5517 102.845) (end 88.485 111.778) (width 0.2) (layer "F.Cu") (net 6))
 (segment (start 101.706 107.824) (end 103.784 107.824) (width 0.2) (layer "F.Cu") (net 6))
 (segment (start 88.485 111.778) (end 93.7972 111.778) (width 0.2) (layer "F.Cu") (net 6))
 (segment (start 99.8052 110.151) (end 99.8052 109.725) (width 0.2) (layer "F.Cu") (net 6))
 (segment (start 106.253 104.88) (end 107.42 104.88) (width 0.2) (layer "F.Cu") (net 6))
 (segment (start 81.2242 114.192) (end 81.2242 119.276) (width 0.2) (layer "F.Cu") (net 1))
 (segment (start 98.6333 96.83) (end 99.8 96.83) (width 0.2) (layer "F.Cu") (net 1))
 (segment (start 86.45 103.49) (end 86.45 102.79) (width 0.2) (layer "F.Cu") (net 1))
 (segment (start 86.45 102.79) (end 85.75 102.79) (width 0.2) (layer "F.Cu") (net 1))
 (segment (start 85.05 101.39) (end 84.35 101.39) (width 0.2) (layer "F.Cu") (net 1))
 (segment (start 86.45 101.39) (end 85.75 101.39) (width 0.2) (layer "F.Cu") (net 1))
 (segment (start 85.75 102.09) (end 84.35 102.09) (width 0.2) (layer "F.Cu") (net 1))
 (segment (start 87.15 104.19) (end 86.45 104.19) (width 0.2) (layer "F.Cu") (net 1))
 (segment (start 87.15 102.09) (end 85.75 102.09) (width 0.2) (layer "F.Cu") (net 1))
 (segment (start 86.45 103.49) (end 85.75 103.49) (width 0.2) (layer "F.Cu") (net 1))
 (segment (start 85.75 103.49) (end 84.35 103.49) (width 0.2) (layer "F.Cu") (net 1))
 (segment (start 85.75 104.19) (end 85.05 104.19) (width 0.2) (layer "F.Cu") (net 1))
 (segment (start 86.45 104.19) (end 85.75 104.19) (width 0.2) (layer "F.Cu") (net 1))
 (segment (start 87.15 103.49) (end 86.45 103.49) (width 0.2) (layer "F.Cu") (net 1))
 (segment (start 93.8 120.78) (end 98.72 120.78) (width 0.2) (layer "F.Cu") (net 1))
 (segment (start 87.15 101.39) (end 86.45 101.39) (width 0.2) (layer "F.Cu") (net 1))
 (segment (start 81.2242 119.276) (end 79.5 121) (width 0.2) (layer "F.Cu") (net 1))
 (segment (start 93.8 120.78) (end 92.8503 121.73) (width 0.2) (layer "F.Cu") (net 1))
 (segment (start 86.45 95.225) (end 78.5 95.225) (width 0.2) (layer "F.Cu") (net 1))
 (segment (start 92.8503 121.73) (end 83.6781 121.73) (width 0.2) (layer "F.Cu") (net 1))
 (segment (start 85.75 102.79) (end 85.05 102.79) (width 0.2) (layer "F.Cu") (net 1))
 (segment (start 98.72 120.78) (end 102.5 117) (width 0.2) (layer "F.Cu") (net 1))
 (segment (start 96 95.225) (end 97.0517 95.225) (width 0.2) (layer "F.Cu") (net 1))
 (segment (start 97.0517 95.225) (end 97.0517 95.2484) (width 0.2) (layer "F.Cu") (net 1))
 (segment (start 83.6781 121.73) (end 81.2242 119.276) (width 0.2) (layer "F.Cu") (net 1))
 (segment (start 87.15 102.79) (end 86.45 102.79) (width 0.2) (layer "F.Cu") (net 1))
 (segment (start 81.535 112.83) (end 81.535 113.882) (width 0.2) (layer "F.Cu") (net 1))
 (segment (start 85.05 104.19) (end 84.35 104.19) (width 0.2) (layer "F.Cu") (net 1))
 (segment (start 85.75 101.39) (end 85.05 101.39) (width 0.2) (layer "F.Cu") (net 1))
 (segment (start 85.05 102.79) (end 84.35 102.79) (width 0.2) (layer "F.Cu") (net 1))
 (segment (start 81.535 113.882) (end 81.2242 114.192) (width 0.2) (layer "F.Cu") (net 1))
 (segment (start 96 95.225) (end 86.45 95.225) (width 0.2) (layer "F.Cu") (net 1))
 (segment (start 97.0517 95.2484) (end 98.6333 96.83) (width 0.2) (layer "F.Cu") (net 1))
 (via (at 86.45 95.225) (size 0.6) (drill 0.3) (layers "F.Cu" "B.Cu") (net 1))
 (segment (start 85.05 102.79) (end 85.05 101.39) (width 0.2) (layer "B.Cu") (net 1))
 (segment (start 99.8 96.83) (end 99.8 104.88) (width 0.2) (layer "B.Cu") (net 1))
 (segment (start 87.15 103.49) (end 87.15 102.09) (width 0.2) (layer "B.Cu") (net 1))
 (segment (start 102.5 117) (end 99.8 114.3) (width 0.2) (layer "B.Cu") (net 1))
 (segment (start 86.45 101.39) (end 86.45 95.225) (width 0.2) (layer "B.Cu") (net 1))
 (segment (start 86.45 104.19) (end 86.45 102.79) (width 0.2) (layer "B.Cu") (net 1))
 (segment (start 99.8 114.3) (end 99.8 104.88) (width 0.2) (layer "B.Cu") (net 1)))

